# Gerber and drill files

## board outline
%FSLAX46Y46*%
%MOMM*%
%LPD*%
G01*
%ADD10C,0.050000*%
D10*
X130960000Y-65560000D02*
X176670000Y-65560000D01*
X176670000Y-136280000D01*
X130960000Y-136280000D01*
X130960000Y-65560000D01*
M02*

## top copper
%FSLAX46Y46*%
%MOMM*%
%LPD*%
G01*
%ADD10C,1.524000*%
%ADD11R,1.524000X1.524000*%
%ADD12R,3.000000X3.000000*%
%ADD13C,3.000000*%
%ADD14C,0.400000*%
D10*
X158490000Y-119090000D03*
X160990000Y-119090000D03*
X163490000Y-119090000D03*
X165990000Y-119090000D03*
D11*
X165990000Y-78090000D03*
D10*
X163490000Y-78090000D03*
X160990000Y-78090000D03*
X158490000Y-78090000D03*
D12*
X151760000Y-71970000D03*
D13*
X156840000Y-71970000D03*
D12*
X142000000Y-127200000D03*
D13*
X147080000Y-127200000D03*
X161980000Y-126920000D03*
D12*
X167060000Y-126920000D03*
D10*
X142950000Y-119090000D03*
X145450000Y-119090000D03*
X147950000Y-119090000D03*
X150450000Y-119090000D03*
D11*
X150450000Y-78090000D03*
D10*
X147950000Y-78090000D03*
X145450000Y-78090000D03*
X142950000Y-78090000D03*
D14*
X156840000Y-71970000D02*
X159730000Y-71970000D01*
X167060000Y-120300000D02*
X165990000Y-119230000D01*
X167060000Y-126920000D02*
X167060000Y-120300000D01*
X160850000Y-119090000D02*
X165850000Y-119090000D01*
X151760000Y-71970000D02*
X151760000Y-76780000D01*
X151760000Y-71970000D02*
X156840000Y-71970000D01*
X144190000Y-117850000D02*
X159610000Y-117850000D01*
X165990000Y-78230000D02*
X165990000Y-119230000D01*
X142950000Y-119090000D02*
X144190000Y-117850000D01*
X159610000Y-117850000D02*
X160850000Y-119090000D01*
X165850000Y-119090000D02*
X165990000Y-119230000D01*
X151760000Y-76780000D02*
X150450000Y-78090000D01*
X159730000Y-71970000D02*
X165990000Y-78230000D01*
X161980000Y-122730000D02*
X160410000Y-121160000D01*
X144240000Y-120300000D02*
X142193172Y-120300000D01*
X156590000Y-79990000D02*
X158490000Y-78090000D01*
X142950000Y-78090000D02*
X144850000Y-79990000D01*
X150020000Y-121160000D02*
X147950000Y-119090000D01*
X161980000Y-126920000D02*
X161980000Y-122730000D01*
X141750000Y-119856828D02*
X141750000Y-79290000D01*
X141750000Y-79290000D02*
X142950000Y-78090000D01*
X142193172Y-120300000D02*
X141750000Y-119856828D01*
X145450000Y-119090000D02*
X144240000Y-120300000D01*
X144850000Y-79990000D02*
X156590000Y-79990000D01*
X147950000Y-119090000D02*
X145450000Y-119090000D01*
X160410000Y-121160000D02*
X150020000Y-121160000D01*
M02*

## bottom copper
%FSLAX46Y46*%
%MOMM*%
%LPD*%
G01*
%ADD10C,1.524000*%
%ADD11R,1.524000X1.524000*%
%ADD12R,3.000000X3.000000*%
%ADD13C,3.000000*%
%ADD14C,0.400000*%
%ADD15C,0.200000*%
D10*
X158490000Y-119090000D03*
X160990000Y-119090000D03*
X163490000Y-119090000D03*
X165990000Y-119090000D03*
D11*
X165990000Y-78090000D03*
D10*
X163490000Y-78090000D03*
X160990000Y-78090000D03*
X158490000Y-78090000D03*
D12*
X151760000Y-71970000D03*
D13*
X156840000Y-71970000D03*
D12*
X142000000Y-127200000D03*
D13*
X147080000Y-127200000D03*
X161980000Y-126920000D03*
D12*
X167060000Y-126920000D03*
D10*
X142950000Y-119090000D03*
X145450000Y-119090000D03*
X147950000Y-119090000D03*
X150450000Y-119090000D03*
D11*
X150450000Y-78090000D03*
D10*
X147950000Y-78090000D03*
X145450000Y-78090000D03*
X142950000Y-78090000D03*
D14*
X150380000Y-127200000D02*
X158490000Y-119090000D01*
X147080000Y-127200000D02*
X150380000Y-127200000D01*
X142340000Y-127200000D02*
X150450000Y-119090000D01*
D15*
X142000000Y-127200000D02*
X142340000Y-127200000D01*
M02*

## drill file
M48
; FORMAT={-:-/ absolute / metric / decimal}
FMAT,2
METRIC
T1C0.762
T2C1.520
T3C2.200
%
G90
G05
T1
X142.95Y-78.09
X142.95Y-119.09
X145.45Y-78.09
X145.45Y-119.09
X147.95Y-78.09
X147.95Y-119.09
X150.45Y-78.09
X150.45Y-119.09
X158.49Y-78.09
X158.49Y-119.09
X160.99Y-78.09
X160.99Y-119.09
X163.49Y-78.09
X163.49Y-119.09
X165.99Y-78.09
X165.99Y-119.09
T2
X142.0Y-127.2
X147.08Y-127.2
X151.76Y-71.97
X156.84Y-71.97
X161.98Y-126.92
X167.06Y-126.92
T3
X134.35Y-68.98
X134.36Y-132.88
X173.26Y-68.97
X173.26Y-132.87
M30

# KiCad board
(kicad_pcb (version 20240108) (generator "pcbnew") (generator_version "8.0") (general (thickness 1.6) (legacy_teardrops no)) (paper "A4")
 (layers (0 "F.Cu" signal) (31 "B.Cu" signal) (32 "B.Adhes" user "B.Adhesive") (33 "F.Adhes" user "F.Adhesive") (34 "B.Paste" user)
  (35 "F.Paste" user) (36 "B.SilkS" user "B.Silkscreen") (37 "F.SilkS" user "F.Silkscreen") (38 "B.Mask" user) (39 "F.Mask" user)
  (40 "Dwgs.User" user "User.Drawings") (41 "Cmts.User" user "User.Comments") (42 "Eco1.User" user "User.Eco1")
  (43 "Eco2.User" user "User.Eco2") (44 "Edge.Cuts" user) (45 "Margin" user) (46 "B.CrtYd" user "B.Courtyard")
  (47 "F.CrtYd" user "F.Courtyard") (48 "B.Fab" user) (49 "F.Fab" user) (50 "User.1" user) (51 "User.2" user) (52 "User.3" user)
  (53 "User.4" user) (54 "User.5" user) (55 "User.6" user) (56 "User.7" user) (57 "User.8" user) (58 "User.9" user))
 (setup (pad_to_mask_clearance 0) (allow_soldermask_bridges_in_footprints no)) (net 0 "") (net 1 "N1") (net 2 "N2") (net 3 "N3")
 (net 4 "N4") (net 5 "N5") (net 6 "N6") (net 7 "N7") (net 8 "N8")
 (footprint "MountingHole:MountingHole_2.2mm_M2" (layer "F.Cu") (at 173.26 132.87)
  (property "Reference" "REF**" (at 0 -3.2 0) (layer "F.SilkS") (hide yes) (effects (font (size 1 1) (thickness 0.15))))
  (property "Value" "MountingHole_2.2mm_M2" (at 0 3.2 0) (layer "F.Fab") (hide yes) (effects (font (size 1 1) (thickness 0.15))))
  (pad "" np_thru_hole circle (at 0 0) (size 2.2 2.2) (drill 2.2) (layers "*.Cu" "*.Mask")))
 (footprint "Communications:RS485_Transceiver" (layer "F.Cu") (at 163.49 97.09 90)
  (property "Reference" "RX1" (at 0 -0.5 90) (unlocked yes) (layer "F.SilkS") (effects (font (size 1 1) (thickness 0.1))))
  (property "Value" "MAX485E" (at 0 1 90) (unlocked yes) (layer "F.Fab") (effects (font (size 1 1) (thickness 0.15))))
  (pad "1" thru_hole circle (at -22 -5 90) (size 1.524 1.524) (drill 0.762) (layers "*.Cu" "*.Mask") (remove_unused_layers no) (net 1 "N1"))
  (pad "2" thru_hole circle (at -22 -2.5 90) (size 1.524 1.524) (drill 0.762) (layers "*.Cu" "*.Mask") (remove_unused_layers no)
   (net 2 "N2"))
  (pad "3" thru_hole circle (at -22 0 90) (size 1.524 1.524) (drill 0.762) (layers "*.Cu" "*.Mask") (remove_unused_layers no) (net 2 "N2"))
  (pad "4" thru_hole circle (at -22 2.5 90) (size 1.524 1.524) (drill 0.762) (layers "*.Cu" "*.Mask") (remove_unused_layers no) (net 2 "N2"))
  (pad "5" thru_hole rect (at 19 2.5 90) (size 1.524 1.524) (drill 0.762) (layers "*.Cu" "*.Mask") (remove_unused_layers no) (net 2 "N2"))
  (pad "6" thru_hole circle (at 19 0 90) (size 1.524 1.524) (drill 0.762) (layers "*.Cu" "*.Mask") (remove_unused_layers no) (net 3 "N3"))
  (pad "7" thru_hole circle (at 19 -2.5 90) (size 1.524 1.524) (drill 0.762) (layers "*.Cu" "*.Mask") (remove_unused_layers no) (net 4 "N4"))
  (pad "8" thru_hole circle (at 19 -5 90) (size 1.524 1.524) (drill 0.762) (layers "*.Cu" "*.Mask") (remove_unused_layers no) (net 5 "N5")))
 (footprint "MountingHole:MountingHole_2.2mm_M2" (layer "F.Cu") (at 134.35 68.98)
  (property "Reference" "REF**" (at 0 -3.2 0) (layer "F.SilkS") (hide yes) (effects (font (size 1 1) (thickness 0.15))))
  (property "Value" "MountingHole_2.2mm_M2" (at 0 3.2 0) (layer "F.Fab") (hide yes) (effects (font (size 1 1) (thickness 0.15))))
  (pad "" np_thru_hole circle (at 0 0) (size 2.2 2.2) (drill 2.2) (layers "*.Cu" "*.Mask")))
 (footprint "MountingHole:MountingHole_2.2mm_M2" (layer "F.Cu") (at 173.26 68.97)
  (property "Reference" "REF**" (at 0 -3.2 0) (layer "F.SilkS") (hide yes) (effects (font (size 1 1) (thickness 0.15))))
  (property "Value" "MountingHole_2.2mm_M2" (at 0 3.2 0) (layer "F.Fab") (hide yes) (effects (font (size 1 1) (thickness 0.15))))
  (pad "" np_thru_hole circle (at 0 0) (size 2.2 2.2) (drill 2.2) (layers "*.Cu" "*.Mask")))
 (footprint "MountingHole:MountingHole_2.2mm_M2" (layer "F.Cu") (at 134.36 132.88)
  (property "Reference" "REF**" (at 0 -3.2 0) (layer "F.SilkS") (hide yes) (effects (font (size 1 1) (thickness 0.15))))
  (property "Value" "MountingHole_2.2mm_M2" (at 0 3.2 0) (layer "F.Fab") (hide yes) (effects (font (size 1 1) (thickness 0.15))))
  (pad "" np_thru_hole circle (at 0 0) (size 2.2 2.2) (drill 2.2) (layers "*.Cu" "*.Mask")))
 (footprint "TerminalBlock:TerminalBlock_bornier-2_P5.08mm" (layer "F.Cu") (at 151.76 71.97)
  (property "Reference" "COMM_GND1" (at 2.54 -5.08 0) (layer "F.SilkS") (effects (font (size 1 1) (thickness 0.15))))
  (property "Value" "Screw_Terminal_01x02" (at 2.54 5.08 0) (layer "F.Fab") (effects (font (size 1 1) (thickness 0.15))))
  (pad "1" thru_hole rect (at 0 0) (size 3 3) (drill 1.52) (layers "*.Cu" "*.Mask") (remove_unused_layers no) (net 2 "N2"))
  (pad "2" thru_hole circle (at 5.08 0) (size 3 3) (drill 1.52) (layers "*.Cu" "*.Mask") (remove_unused_layers no) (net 2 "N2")))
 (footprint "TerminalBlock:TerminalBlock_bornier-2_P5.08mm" (layer "F.Cu") (at 142 127.2)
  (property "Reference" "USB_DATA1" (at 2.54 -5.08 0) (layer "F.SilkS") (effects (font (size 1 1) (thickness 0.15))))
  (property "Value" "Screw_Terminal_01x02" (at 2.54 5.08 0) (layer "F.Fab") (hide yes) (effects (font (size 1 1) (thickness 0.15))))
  (pad "1" thru_hole rect (at 0 0) (size 3 3) (drill 1.52) (layers "*.Cu" "*.Mask") (remove_unused_layers no) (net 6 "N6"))
  (pad "2" thru_hole circle (at 5.08 0) (size 3 3) (drill 1.52) (layers "*.Cu" "*.Mask") (remove_unused_layers no) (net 1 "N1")))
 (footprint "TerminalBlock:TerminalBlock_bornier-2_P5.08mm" (layer "F.Cu") (at 161.98 126.92)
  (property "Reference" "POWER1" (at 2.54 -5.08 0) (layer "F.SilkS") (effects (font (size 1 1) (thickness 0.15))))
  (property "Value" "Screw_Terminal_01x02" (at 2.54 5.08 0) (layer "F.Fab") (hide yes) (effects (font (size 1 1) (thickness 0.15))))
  (pad "1" thru_hole circle (at 0 0) (size 3 3) (drill 1.52) (layers "*.Cu" "*.Mask") (remove_unused_layers no) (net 5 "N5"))
  (pad "2" thru_hole rect (at 5.08 0) (size 3 3) (drill 1.52) (layers "*.Cu" "*.Mask") (remove_unused_layers no) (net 2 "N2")))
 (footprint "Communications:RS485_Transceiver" (layer "F.Cu") (at 147.95 97.09 90)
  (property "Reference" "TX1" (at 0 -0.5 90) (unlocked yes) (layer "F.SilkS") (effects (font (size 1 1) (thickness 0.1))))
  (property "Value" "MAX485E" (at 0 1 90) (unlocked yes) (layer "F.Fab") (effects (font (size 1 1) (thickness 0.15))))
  (pad "1" thru_hole circle (at -22 -5 90) (size 1.524 1.524) (drill 0.762) (layers "*.Cu" "*.Mask") (remove_unused_layers no) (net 2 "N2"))
  (pad "2" thru_hole circle (at -22 -2.5 90) (size 1.524 1.524) (drill 0.762) (layers "*.Cu" "*.Mask") (remove_unused_layers no)
   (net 5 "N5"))
  (pad "3" thru_hole circle (at -22 0 90) (size 1.524 1.524) (drill 0.762) (layers "*.Cu" "*.Mask") (remove_unused_layers no) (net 5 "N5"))
  (pad "4" thru_hole circle (at -22 2.5 90) (size 1.524 1.524) (drill 0.762) (layers "*.Cu" "*.Mask") (remove_unused_layers no) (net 6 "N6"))
  (pad "5" thru_hole rect (at 19 2.5 90) (size 1.524 1.524) (drill 0.762) (layers "*.Cu" "*.Mask") (remove_unused_layers no) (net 2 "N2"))
  (pad "6" thru_hole circle (at 19 0 90) (size 1.524 1.524) (drill 0.762) (layers "*.Cu" "*.Mask") (remove_unused_layers no) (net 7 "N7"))
  (pad "7" thru_hole circle (at 19 -2.5 90) (size 1.524 1.524) (drill 0.762) (layers "*.Cu" "*.Mask") (remove_unused_layers no) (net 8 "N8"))
  (pad "8" thru_hole circle (at 19 -5 90) (size 1.524 1.524) (drill 0.762) (layers "*.Cu" "*.Mask") (remove_unused_layers no) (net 5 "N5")))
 (gr_rect (start 130.96 65.56) (end 176.67 136.28) (stroke (width 0.05) (type default)) (fill none) (layer "Edge.Cuts"))
 (segment (start 156.84 71.97) (end 159.73 71.97) (width 0.4) (layer "F.Cu") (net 2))
 (segment (start 167.06 120.3) (end 165.99 119.23) (width 0.4) (layer "F.Cu") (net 2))
 (segment (start 167.06 126.92) (end 167.06 120.3) (width 0.4) (layer "F.Cu") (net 2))
 (segment (start 160.85 119.09) (end 165.85 119.09) (width 0.4) (layer "F.Cu") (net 2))
 (segment (start 151.76 71.97) (end 151.76 76.78) (width 0.4) (layer "F.Cu") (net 2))
 (segment (start 151.76 71.97) (end 156.84 71.97) (width 0.4) (layer "F.Cu") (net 2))
 (segment (start 144.19 117.85) (end 159.61 117.85) (width 0.4) (layer "F.Cu") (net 2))
 (segment (start 165.99 78.23) (end 165.99 119.23) (width 0.4) (layer "F.Cu") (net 2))
 (segment (start 142.95 119.09) (end 144.19 117.85) (width 0.4) (layer "F.Cu") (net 2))
 (segment (start 159.61 117.85) (end 160.85 119.09) (width 0.4) (layer "F.Cu") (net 2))
 (segment (start 165.85 119.09) (end 165.99 119.23) (width 0.4) (layer "F.Cu") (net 2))
 (segment (start 151.76 76.78) (end 150.45 78.09) (width 0.4) (layer "F.Cu") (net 2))
 (segment (start 159.73 71.97) (end 165.99 78.23) (width 0.4) (layer "F.Cu") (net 2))
 (segment (start 161.98 122.73) (end 160.41 121.16) (width 0.4) (layer "F.Cu") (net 5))
 (segment (start 144.24 120.3) (end 142.193172 120.3) (width 0.4) (layer "F.Cu") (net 5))
 (segment (start 156.59 79.99) (end 158.49 78.09) (width 0.4) (layer "F.Cu") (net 5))
 (segment (start 142.95 78.09) (end 144.85 79.99) (width 0.4) (layer "F.Cu") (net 5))
 (segment (start 150.02 121.16) (end 147.95 119.09) (width 0.4) (layer "F.Cu") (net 5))
 (segment (start 161.98 126.92) (end 161.98 122.73) (width 0.4) (layer "F.Cu") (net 5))
 (segment (start 141.75 119.856828) (end 141.75 79.29) (width 0.4) (layer "F.Cu") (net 5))
 (segment (start 141.75 79.29) (end 142.95 78.09) (width 0.4) (layer "F.Cu") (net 5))
 (segment (start 142.193172 120.3) (end 141.75 119.856828) (width 0.4) (layer "F.Cu") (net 5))
 (segment (start 145.45 119.09) (end 144.24 120.3) (width 0.4) (layer "F.Cu") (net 5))
 (segment (start 144.85 79.99) (end 156.59 79.99) (width 0.4) (layer "F.Cu") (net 5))
 (segment (start 147.95 119.09) (end 145.45 119.09) (width 0.4) (layer "F.Cu") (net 5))
 (segment (start 160.41 121.16) (end 150.02 121.16) (width 0.4) (layer "F.Cu") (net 5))
 (segment (start 150.38 127.2) (end 158.49 119.09) (width 0.4) (layer "B.Cu") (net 1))
 (segment (start 147.08 127.2) (end 150.38 127.2) (width 0.4) (layer "B.Cu") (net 1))
 (segment (start 142.34 127.2) (end 150.45 119.09) (width 0.4) (layer "B.Cu") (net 6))
 (segment (start 142 127.2) (end 142.34 127.2) (width 0.2) (layer "B.Cu") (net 6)))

